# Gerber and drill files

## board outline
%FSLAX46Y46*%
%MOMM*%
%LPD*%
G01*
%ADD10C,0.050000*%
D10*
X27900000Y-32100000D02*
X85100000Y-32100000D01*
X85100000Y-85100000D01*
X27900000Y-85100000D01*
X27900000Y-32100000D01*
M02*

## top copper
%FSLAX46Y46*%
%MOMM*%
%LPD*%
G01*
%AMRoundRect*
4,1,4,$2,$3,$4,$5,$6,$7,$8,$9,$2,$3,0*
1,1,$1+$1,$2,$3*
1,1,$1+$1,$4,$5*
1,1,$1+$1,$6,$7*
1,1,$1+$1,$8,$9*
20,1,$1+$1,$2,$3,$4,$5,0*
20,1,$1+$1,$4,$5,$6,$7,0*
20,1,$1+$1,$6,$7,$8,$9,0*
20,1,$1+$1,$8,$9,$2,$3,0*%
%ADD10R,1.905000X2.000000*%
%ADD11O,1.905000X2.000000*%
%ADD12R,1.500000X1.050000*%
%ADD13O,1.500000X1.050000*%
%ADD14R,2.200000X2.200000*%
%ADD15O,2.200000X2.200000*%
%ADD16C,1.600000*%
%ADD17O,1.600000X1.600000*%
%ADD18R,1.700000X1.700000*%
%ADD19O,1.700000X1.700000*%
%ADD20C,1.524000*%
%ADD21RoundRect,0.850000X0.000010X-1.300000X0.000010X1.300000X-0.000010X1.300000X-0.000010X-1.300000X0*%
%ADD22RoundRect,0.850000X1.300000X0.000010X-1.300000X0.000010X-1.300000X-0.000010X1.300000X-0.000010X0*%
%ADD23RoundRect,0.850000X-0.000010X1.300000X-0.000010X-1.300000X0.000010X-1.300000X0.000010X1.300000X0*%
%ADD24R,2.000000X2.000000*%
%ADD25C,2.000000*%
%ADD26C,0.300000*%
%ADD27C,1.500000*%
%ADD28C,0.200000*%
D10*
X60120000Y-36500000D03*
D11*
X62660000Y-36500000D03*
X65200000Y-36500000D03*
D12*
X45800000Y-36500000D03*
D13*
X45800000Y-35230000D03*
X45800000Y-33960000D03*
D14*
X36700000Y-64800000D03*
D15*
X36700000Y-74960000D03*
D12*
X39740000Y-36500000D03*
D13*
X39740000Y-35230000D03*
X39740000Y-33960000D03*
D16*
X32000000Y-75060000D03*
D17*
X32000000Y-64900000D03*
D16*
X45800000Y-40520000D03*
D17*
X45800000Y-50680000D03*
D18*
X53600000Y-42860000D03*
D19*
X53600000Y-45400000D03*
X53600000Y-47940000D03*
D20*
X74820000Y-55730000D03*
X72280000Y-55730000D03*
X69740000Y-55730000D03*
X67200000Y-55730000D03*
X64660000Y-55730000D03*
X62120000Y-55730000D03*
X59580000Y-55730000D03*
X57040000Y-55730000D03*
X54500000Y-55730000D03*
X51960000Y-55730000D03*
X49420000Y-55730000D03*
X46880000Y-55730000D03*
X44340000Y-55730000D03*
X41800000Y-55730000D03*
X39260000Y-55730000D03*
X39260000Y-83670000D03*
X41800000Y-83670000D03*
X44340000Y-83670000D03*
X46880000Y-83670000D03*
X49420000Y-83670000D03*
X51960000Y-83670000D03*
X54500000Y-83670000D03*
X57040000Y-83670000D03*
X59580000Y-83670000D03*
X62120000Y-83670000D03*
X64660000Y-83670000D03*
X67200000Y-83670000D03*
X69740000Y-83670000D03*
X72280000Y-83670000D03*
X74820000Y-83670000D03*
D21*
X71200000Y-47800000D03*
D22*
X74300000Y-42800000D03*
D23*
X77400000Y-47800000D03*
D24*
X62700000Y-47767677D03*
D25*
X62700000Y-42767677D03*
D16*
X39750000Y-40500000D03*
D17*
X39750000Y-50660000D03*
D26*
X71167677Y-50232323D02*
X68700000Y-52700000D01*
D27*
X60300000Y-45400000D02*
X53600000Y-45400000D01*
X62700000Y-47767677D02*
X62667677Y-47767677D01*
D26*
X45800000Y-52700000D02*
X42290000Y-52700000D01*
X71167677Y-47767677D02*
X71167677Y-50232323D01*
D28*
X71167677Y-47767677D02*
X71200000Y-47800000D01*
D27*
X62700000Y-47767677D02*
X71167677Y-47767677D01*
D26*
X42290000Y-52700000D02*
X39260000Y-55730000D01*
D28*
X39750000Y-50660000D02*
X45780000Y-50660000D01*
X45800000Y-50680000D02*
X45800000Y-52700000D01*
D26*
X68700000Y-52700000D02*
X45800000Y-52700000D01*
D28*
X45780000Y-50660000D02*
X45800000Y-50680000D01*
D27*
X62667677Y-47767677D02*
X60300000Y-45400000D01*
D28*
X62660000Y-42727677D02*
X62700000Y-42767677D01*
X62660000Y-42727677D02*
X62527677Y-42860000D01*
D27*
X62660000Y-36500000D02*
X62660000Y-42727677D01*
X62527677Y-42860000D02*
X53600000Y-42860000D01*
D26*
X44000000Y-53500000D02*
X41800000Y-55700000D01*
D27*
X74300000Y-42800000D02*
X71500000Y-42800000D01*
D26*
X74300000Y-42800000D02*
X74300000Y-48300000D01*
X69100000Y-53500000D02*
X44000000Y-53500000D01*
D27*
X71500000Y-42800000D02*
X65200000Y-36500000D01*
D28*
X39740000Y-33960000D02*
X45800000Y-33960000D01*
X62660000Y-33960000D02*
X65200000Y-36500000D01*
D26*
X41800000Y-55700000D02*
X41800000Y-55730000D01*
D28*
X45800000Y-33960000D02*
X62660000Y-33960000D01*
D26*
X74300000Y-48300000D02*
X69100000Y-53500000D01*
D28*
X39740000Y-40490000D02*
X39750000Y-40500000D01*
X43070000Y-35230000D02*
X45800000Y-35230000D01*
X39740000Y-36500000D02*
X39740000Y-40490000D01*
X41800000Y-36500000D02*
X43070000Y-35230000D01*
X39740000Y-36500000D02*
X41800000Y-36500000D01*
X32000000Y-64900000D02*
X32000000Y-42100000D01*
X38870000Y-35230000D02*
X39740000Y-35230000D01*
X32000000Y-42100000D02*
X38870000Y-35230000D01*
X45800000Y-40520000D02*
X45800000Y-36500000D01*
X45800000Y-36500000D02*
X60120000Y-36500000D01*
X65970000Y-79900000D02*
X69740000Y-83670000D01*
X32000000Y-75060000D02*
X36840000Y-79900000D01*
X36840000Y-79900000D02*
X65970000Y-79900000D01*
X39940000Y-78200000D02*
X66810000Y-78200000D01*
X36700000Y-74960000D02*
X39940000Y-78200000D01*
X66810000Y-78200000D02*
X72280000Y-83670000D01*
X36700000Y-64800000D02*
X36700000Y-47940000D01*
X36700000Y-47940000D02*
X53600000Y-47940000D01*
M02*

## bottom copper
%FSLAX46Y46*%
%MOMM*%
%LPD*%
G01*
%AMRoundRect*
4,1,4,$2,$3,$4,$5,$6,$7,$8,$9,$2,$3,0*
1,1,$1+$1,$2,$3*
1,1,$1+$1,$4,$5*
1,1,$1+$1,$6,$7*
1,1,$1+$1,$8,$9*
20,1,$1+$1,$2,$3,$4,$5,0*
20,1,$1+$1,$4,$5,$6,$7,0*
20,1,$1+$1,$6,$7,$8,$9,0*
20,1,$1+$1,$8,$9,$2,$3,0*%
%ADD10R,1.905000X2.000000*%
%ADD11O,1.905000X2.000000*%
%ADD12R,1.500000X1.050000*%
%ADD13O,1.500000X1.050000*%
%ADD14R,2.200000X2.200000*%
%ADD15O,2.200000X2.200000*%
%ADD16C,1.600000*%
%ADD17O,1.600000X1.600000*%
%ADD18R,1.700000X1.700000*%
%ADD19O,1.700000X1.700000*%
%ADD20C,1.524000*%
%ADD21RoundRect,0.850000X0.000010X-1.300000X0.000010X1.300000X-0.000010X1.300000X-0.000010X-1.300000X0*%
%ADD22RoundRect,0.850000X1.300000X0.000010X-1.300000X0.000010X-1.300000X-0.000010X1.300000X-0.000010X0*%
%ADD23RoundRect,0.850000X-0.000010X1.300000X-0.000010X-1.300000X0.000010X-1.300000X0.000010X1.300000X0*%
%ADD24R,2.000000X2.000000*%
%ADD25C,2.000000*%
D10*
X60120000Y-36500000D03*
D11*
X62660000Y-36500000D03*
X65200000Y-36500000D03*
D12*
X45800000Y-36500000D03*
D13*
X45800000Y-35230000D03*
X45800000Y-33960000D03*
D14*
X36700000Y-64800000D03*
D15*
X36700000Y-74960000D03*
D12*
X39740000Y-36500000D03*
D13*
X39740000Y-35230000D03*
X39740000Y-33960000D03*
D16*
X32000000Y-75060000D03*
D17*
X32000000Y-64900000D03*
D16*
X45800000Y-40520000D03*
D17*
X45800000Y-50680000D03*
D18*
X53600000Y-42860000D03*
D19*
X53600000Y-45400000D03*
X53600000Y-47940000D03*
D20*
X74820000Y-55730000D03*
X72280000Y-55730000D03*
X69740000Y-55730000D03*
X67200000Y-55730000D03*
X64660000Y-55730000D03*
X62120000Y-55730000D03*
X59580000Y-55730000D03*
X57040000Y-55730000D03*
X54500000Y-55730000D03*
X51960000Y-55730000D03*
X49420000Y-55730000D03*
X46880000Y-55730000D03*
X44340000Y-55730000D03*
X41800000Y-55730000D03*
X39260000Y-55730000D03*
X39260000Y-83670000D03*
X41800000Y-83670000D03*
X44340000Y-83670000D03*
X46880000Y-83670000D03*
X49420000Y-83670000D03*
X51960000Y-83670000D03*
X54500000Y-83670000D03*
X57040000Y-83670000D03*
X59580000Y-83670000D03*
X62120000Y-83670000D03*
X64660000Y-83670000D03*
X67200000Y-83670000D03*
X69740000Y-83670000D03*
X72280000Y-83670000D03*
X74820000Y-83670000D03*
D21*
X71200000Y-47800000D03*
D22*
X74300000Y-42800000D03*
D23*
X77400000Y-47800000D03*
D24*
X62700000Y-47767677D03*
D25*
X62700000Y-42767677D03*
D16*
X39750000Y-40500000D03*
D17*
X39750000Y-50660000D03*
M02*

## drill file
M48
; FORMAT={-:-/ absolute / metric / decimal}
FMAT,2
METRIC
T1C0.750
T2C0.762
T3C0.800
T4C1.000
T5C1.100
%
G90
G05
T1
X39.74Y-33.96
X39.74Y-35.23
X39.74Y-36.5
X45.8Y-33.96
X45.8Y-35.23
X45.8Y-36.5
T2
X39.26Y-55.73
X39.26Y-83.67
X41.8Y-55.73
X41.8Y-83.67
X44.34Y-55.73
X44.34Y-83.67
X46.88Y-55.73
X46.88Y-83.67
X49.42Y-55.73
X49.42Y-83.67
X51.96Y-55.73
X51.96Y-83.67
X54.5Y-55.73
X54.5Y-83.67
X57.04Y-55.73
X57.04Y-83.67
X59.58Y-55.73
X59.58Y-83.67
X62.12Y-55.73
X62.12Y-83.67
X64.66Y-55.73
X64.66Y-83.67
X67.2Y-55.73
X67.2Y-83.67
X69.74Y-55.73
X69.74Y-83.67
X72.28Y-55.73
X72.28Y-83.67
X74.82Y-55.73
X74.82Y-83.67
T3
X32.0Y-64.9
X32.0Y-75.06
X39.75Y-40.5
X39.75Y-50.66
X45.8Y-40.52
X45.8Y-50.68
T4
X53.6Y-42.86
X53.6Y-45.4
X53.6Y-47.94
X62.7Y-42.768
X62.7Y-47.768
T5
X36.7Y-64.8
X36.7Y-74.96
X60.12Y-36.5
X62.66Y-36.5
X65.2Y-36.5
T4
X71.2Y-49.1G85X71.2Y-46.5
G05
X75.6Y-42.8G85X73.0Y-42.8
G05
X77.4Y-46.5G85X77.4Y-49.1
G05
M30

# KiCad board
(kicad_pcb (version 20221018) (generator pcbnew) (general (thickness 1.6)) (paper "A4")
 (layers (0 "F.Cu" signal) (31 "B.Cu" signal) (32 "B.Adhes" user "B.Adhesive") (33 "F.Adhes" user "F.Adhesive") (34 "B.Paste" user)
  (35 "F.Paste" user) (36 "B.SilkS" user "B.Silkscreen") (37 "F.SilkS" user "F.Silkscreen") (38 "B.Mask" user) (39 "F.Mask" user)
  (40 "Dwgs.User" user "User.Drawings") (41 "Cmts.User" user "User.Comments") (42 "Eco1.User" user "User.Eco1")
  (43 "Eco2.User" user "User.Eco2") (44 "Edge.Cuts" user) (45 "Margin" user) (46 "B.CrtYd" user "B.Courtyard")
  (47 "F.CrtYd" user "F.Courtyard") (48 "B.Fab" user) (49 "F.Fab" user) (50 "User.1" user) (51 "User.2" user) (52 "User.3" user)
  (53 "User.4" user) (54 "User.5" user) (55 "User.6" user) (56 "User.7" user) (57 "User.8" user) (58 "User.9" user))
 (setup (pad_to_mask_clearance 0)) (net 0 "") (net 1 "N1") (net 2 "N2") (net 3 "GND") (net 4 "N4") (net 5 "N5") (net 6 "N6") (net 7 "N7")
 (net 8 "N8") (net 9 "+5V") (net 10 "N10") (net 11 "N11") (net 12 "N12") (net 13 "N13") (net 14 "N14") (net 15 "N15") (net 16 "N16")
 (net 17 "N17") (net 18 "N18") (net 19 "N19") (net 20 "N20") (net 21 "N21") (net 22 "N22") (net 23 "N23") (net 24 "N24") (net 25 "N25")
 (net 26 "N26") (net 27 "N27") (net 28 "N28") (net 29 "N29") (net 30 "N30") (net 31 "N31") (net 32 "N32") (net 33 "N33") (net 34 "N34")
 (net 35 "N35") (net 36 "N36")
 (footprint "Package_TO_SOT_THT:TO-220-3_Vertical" (layer "F.Cu") (at 60.12 36.5)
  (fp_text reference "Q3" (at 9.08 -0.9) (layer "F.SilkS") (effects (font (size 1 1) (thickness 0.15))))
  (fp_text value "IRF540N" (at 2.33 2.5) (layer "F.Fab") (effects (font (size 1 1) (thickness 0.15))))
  (pad "1" thru_hole rect (at 0 0) (size 1.905 2) (drill 1.1) (layers "*.Cu" "*.Mask") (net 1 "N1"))
  (pad "2" thru_hole oval (at 2.54 0) (size 1.905 2) (drill 1.1) (layers "*.Cu" "*.Mask") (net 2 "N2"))
  (pad "3" thru_hole oval (at 5.08 0) (size 1.905 2) (drill 1.1) (layers "*.Cu" "*.Mask") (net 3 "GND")))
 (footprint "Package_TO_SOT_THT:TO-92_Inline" (layer "F.Cu") (at 45.8 36.5 90)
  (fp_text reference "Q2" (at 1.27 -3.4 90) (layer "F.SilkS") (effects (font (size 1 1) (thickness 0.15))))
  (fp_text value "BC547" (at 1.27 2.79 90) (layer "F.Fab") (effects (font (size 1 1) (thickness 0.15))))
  (pad "1" thru_hole rect (at 0 0 90) (size 1.05 1.5) (drill 0.75) (layers "*.Cu" "*.Mask") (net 1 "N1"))
  (pad "2" thru_hole oval (at 1.27 0 90) (size 1.05 1.5) (drill 0.75) (layers "*.Cu" "*.Mask") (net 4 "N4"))
  (pad "3" thru_hole oval (at 2.54 0 90) (size 1.05 1.5) (drill 0.75) (layers "*.Cu" "*.Mask") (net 3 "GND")))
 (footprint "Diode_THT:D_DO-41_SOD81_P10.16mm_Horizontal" (layer "F.Cu") (at 36.7 64.8 -90)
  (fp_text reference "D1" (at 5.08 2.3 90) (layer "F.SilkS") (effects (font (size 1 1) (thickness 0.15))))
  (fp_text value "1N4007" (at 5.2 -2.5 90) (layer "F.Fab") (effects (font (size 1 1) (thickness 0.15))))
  (pad "1" thru_hole rect (at 0 0 270) (size 2.2 2.2) (drill 1.1) (layers "*.Cu" "*.Mask") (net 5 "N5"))
  (pad "2" thru_hole oval (at 10.16 0 270) (size 2.2 2.2) (drill 1.1) (layers "*.Cu" "*.Mask") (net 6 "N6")))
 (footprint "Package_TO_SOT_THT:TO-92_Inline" (layer "F.Cu") (at 39.74 36.5 90)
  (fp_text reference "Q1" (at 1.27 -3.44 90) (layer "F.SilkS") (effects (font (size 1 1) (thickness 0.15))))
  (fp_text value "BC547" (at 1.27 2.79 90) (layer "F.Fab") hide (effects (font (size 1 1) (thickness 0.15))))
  (pad "1" thru_hole rect (at 0 0 90) (size 1.05 1.5) (drill 0.75) (layers "*.Cu" "*.Mask") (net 4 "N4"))
  (pad "2" thru_hole oval (at 1.27 0 90) (size 1.05 1.5) (drill 0.75) (layers "*.Cu" "*.Mask") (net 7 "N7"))
  (pad "3" thru_hole oval (at 2.54 0 90) (size 1.05 1.5) (drill 0.75) (layers "*.Cu" "*.Mask") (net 3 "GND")))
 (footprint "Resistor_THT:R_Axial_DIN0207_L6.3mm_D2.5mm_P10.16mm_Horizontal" (layer "F.Cu") (at 32 75.06 90)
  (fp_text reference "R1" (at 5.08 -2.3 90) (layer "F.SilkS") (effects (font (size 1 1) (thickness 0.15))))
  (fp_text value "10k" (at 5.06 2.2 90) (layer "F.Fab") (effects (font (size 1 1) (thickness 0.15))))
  (pad "1" thru_hole circle (at 0 0 90) (size 1.6 1.6) (drill 0.8) (layers "*.Cu" "*.Mask") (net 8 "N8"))
  (pad "2" thru_hole oval (at 10.16 0 90) (size 1.6 1.6) (drill 0.8) (layers "*.Cu" "*.Mask") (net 7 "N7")))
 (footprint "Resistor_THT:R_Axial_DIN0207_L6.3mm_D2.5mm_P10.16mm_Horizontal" (layer "F.Cu") (at 45.8 40.52 -90)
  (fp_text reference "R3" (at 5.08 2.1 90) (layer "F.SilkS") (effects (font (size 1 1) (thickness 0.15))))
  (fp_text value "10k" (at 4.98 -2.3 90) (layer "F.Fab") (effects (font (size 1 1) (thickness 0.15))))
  (pad "1" thru_hole circle (at 0 0 270) (size 1.6 1.6) (drill 0.8) (layers "*.Cu" "*.Mask") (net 1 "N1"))
  (pad "2" thru_hole oval (at 10.16 0 270) (size 1.6 1.6) (drill 0.8) (layers "*.Cu" "*.Mask") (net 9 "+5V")))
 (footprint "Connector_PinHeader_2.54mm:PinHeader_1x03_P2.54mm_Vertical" (layer "F.Cu") (at 53.6 42.86)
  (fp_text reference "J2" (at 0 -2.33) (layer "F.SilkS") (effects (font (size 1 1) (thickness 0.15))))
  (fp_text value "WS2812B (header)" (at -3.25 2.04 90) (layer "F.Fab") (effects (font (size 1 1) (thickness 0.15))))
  (pad "1" thru_hole rect (at 0 0) (size 1.7 1.7) (drill 1) (layers "*.Cu" "*.Mask") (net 2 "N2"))
  (pad "2" thru_hole oval (at 0 2.54) (size 1.7 1.7) (drill 1) (layers "*.Cu" "*.Mask") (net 9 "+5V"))
  (pad "3" thru_hole oval (at 0 5.08) (size 1.7 1.7) (drill 1) (layers "*.Cu" "*.Mask") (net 5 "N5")))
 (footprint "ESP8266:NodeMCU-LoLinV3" (layer "F.Cu") (at 54.5 69.7 -90)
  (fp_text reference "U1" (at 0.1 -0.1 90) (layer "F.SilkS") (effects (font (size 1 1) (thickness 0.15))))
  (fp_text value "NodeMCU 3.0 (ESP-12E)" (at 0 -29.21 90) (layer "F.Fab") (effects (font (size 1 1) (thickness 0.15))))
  (pad "1" thru_hole circle (at -13.97 -20.32 270) (size 1.524 1.524) (drill 0.762) (layers "*.Cu" "*.Mask" "F.SilkS") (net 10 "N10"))
  (pad "2" thru_hole circle (at -13.97 -17.78 270) (size 1.524 1.524) (drill 0.762) (layers "*.Cu" "*.Mask" "F.SilkS") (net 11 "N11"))
  (pad "3" thru_hole circle (at -13.97 -15.24 270) (size 1.524 1.524) (drill 0.762) (layers "*.Cu" "*.Mask" "F.SilkS") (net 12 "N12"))
  (pad "4" thru_hole circle (at -13.97 -12.7 270) (size 1.524 1.524) (drill 0.762) (layers "*.Cu" "*.Mask" "F.SilkS") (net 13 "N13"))
  (pad "5" thru_hole circle (at -13.97 -10.16 270) (size 1.524 1.524) (drill 0.762) (layers "*.Cu" "*.Mask" "F.SilkS") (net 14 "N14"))
  (pad "6" thru_hole circle (at -13.97 -7.62 270) (size 1.524 1.524) (drill 0.762) (layers "*.Cu" "*.Mask" "F.SilkS") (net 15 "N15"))
  (pad "7" thru_hole circle (at -13.97 -5.08 270) (size 1.524 1.524) (drill 0.762) (layers "*.Cu" "*.Mask" "F.SilkS") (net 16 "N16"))
  (pad "8" thru_hole circle (at -13.97 -2.54 270) (size 1.524 1.524) (drill 0.762) (layers "*.Cu" "*.Mask" "F.SilkS") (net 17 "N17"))
  (pad "9" thru_hole circle (at -13.97 0 270) (size 1.524 1.524) (drill 0.762) (layers "*.Cu" "*.Mask" "F.SilkS") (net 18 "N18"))
  (pad "10" thru_hole circle (at -13.97 2.54 270) (size 1.524 1.524) (drill 0.762) (layers "*.Cu" "*.Mask" "F.SilkS") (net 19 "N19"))
  (pad "11" thru_hole circle (at -13.97 5.08 270) (size 1.524 1.524) (drill 0.762) (layers "*.Cu" "*.Mask" "F.SilkS") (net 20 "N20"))
  (pad "12" thru_hole circle (at -13.97 7.62 270) (size 1.524 1.524) (drill 0.762) (layers "*.Cu" "*.Mask" "F.SilkS") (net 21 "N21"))
  (pad "13" thru_hole circle (at -13.97 10.16 270) (size 1.524 1.524) (drill 0.762) (layers "*.Cu" "*.Mask" "F.SilkS") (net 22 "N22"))
  (pad "14" thru_hole circle (at -13.97 12.7 270) (size 1.524 1.524) (drill 0.762) (layers "*.Cu" "*.Mask" "F.SilkS") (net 3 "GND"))
  (pad "15" thru_hole circle (at -13.97 15.24 270) (size 1.524 1.524) (drill 0.762) (layers "*.Cu" "*.Mask" "F.SilkS") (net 9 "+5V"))
  (pad "16" thru_hole circle (at 13.97 15.24 270) (size 1.524 1.524) (drill 0.762) (layers "*.Cu" "*.Mask" "F.SilkS") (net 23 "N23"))
  (pad "17" thru_hole circle (at 13.97 12.7 270) (size 1.524 1.524) (drill 0.762) (layers "*.Cu" "*.Mask" "F.SilkS") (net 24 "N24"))
  (pad "18" thru_hole circle (at 13.97 10.16 270) (size 1.524 1.524) (drill 0.762) (layers "*.Cu" "*.Mask" "F.SilkS") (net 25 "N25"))
  (pad "19" thru_hole circle (at 13.97 7.62 270) (size 1.524 1.524) (drill 0.762) (layers "*.Cu" "*.Mask" "F.SilkS") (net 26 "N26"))
  (pad "20" thru_hole circle (at 13.97 5.08 270) (size 1.524 1.524) (drill 0.762) (layers "*.Cu" "*.Mask" "F.SilkS") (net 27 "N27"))
  (pad "21" thru_hole circle (at 13.97 2.54 270) (size 1.524 1.524) (drill 0.762) (layers "*.Cu" "*.Mask" "F.SilkS") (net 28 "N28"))
  (pad "22" thru_hole circle (at 13.97 0 270) (size 1.524 1.524) (drill 0.762) (layers "*.Cu" "*.Mask" "F.SilkS") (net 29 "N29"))
  (pad "23" thru_hole circle (at 13.97 -2.54 270) (size 1.524 1.524) (drill 0.762) (layers "*.Cu" "*.Mask" "F.SilkS") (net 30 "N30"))
  (pad "24" thru_hole circle (at 13.97 -5.08 270) (size 1.524 1.524) (drill 0.762) (layers "*.Cu" "*.Mask" "F.SilkS") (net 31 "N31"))
  (pad "25" thru_hole circle (at 13.97 -7.62 270) (size 1.524 1.524) (drill 0.762) (layers "*.Cu" "*.Mask" "F.SilkS") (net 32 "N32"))
  (pad "26" thru_hole circle (at 13.97 -10.16 270) (size 1.524 1.524) (drill 0.762) (layers "*.Cu" "*.Mask" "F.SilkS") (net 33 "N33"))
  (pad "27" thru_hole circle (at 13.97 -12.7 270) (size 1.524 1.524) (drill 0.762) (layers "*.Cu" "*.Mask" "F.SilkS") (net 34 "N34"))
  (pad "28" thru_hole circle (at 13.97 -15.24 270) (size 1.524 1.524) (drill 0.762) (layers "*.Cu" "*.Mask" "F.SilkS") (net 8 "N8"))
  (pad "29" thru_hole circle (at 13.97 -17.78 270) (size 1.524 1.524) (drill 0.762) (layers "*.Cu" "*.Mask" "F.SilkS") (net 6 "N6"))
  (pad "30" thru_hole circle (at 13.97 -20.32 270) (size 1.524 1.524) (drill 0.762) (layers "*.Cu" "*.Mask" "F.SilkS") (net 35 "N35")))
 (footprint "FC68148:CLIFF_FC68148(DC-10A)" (layer "F.Cu") (at 77.4 47.8 90)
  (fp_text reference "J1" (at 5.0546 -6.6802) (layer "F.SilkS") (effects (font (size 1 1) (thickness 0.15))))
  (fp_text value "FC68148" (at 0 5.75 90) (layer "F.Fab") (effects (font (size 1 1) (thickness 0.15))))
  (pad "1" thru_hole roundrect (at 0 -6.2 90) (size 4.3 1.7) (drill oval 3.6 1) (layers "*.Cu" "*.Mask") (roundrect_rratio 0.5)
   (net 9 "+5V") (solder_mask_margin 0.102))
  (pad "2" thru_hole roundrect (at 5 -3.1 180) (size 4.3 1.7) (drill oval 3.6 1) (layers "*.Cu" "*.Mask") (roundrect_rratio 0.5)
   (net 3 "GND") (solder_mask_margin 0.102))
  (pad "3" thru_hole roundrect (at 0 0 270) (size 4.3 1.7) (drill oval 3.6 1) (layers "*.Cu" "*.Mask") (roundrect_rratio 0.5) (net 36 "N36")
   (solder_mask_margin 0.102)))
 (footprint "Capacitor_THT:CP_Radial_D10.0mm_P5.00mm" (layer "F.Cu") (at 62.7 47.767677 90)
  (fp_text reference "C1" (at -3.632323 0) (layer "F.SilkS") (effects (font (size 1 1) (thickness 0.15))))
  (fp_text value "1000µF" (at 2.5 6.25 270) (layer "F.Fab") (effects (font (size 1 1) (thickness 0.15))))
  (pad "1" thru_hole rect (at 0 0 90) (size 2 2) (drill 1) (layers "*.Cu" "*.Mask") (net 9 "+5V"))
  (pad "2" thru_hole circle (at 5 0 90) (size 2 2) (drill 1) (layers "*.Cu" "*.Mask") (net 2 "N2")))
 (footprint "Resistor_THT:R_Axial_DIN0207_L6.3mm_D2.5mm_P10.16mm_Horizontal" (layer "F.Cu") (at 39.75 40.5 -90)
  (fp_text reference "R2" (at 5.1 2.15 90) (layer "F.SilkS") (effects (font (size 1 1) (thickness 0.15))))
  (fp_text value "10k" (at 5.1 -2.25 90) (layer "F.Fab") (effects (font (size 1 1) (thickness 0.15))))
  (pad "1" thru_hole circle (at 0 0 270) (size 1.6 1.6) (drill 0.8) (layers "*.Cu" "*.Mask") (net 4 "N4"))
  (pad "2" thru_hole oval (at 10.16 0 270) (size 1.6 1.6) (drill 0.8) (layers "*.Cu" "*.Mask") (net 9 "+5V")))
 (gr_rect (start 27.9 32.1) (end 85.1 85.1) (stroke (width 0.05) (type default)) (fill none) (layer "Edge.Cuts"))
 (segment (start 71.167677 50.232323) (end 68.7 52.7) (width 0.3) (layer "F.Cu") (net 9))
 (segment (start 60.3 45.4) (end 53.6 45.4) (width 1.5) (layer "F.Cu") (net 9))
 (segment (start 62.7 47.767677) (end 62.667677 47.767677) (width 1.5) (layer "F.Cu") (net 9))
 (segment (start 45.8 52.7) (end 42.29 52.7) (width 0.3) (layer "F.Cu") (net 9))
 (segment (start 71.167677 47.767677) (end 71.167677 50.232323) (width 0.3) (layer "F.Cu") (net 9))
 (segment (start 71.167677 47.767677) (end 71.2 47.8) (width 0.2) (layer "F.Cu") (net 9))
 (segment (start 62.7 47.767677) (end 71.167677 47.767677) (width 1.5) (layer "F.Cu") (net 9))
 (segment (start 42.29 52.7) (end 39.26 55.73) (width 0.3) (layer "F.Cu") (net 9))
 (segment (start 39.75 50.66) (end 45.78 50.66) (width 0.2) (layer "F.Cu") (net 9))
 (segment (start 45.8 50.68) (end 45.8 52.7) (width 0.2) (layer "F.Cu") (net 9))
 (segment (start 68.7 52.7) (end 45.8 52.7) (width 0.3) (layer "F.Cu") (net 9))
 (segment (start 45.78 50.66) (end 45.8 50.68) (width 0.2) (layer "F.Cu") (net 9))
 (segment (start 62.667677 47.767677) (end 60.3 45.4) (width 1.5) (layer "F.Cu") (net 9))
 (segment (start 62.66 42.727677) (end 62.7 42.767677) (width 0.2) (layer "F.Cu") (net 2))
 (segment (start 62.66 42.727677) (end 62.527677 42.86) (width 0.2) (layer "F.Cu") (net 2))
 (segment (start 62.66 36.5) (end 62.66 42.727677) (width 1.5) (layer "F.Cu") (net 2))
 (segment (start 62.527677 42.86) (end 53.6 42.86) (width 1.5) (layer "F.Cu") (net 2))
 (segment (start 44 53.5) (end 41.8 55.7) (width 0.3) (layer "F.Cu") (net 3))
 (segment (start 74.3 42.8) (end 71.5 42.8) (width 1.5) (layer "F.Cu") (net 3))
 (segment (start 74.3 42.8) (end 74.3 48.3) (width 0.3) (layer "F.Cu") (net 3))
 (segment (start 69.1 53.5) (end 44 53.5) (width 0.3) (layer "F.Cu") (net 3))
 (segment (start 71.5 42.8) (end 65.2 36.5) (width 1.5) (layer "F.Cu") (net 3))
 (segment (start 39.74 33.96) (end 45.8 33.96) (width 0.2) (layer "F.Cu") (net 3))
 (segment (start 62.66 33.96) (end 65.2 36.5) (width 0.2) (layer "F.Cu") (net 3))
 (segment (start 41.8 55.7) (end 41.8 55.73) (width 0.3) (layer "F.Cu") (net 3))
 (segment (start 45.8 33.96) (end 62.66 33.96) (width 0.2) (layer "F.Cu") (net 3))
 (segment (start 74.3 48.3) (end 69.1 53.5) (width 0.3) (layer "F.Cu") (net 3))
 (segment (start 39.74 40.49) (end 39.75 40.5) (width 0.2) (layer "F.Cu") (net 4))
 (segment (start 43.07 35.23) (end 45.8 35.23) (width 0.2) (layer "F.Cu") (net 4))
 (segment (start 39.74 36.5) (end 39.74 40.49) (width 0.2) (layer "F.Cu") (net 4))
 (segment (start 41.8 36.5) (end 43.07 35.23) (width 0.2) (layer "F.Cu") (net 4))
 (segment (start 39.74 36.5) (end 41.8 36.5) (width 0.2) (layer "F.Cu") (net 4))
 (segment (start 32 64.9) (end 32 42.1) (width 0.2) (layer "F.Cu") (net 7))
 (segment (start 38.87 35.23) (end 39.74 35.23) (width 0.2) (layer "F.Cu") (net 7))
 (segment (start 32 42.1) (end 38.87 35.23) (width 0.2) (layer "F.Cu") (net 7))
 (segment (start 45.8 40.52) (end 45.8 36.5) (width 0.2) (layer "F.Cu") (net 1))
 (segment (start 45.8 36.5) (end 60.12 36.5) (width 0.2) (layer "F.Cu") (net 1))
 (segment (start 65.97 79.9) (end 69.74 83.67) (width 0.2) (layer "F.Cu") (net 8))
 (segment (start 32 75.06) (end 36.84 79.9) (width 0.2) (layer "F.Cu") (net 8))
 (segment (start 36.84 79.9) (end 65.97 79.9) (width 0.2) (layer "F.Cu") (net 8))
 (segment (start 39.94 78.2) (end 66.81 78.2) (width 0.2) (layer "F.Cu") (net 6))
 (segment (start 36.7 74.96) (end 39.94 78.2) (width 0.2) (layer "F.Cu") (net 6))
 (segment (start 66.81 78.2) (end 72.28 83.67) (width 0.2) (layer "F.Cu") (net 6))
 (segment (start 36.7 64.8) (end 36.7 47.94) (width 0.2) (layer "F.Cu") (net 5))
 (segment (start 36.7 47.94) (end 53.6 47.94) (width 0.2) (layer "F.Cu") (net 5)))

